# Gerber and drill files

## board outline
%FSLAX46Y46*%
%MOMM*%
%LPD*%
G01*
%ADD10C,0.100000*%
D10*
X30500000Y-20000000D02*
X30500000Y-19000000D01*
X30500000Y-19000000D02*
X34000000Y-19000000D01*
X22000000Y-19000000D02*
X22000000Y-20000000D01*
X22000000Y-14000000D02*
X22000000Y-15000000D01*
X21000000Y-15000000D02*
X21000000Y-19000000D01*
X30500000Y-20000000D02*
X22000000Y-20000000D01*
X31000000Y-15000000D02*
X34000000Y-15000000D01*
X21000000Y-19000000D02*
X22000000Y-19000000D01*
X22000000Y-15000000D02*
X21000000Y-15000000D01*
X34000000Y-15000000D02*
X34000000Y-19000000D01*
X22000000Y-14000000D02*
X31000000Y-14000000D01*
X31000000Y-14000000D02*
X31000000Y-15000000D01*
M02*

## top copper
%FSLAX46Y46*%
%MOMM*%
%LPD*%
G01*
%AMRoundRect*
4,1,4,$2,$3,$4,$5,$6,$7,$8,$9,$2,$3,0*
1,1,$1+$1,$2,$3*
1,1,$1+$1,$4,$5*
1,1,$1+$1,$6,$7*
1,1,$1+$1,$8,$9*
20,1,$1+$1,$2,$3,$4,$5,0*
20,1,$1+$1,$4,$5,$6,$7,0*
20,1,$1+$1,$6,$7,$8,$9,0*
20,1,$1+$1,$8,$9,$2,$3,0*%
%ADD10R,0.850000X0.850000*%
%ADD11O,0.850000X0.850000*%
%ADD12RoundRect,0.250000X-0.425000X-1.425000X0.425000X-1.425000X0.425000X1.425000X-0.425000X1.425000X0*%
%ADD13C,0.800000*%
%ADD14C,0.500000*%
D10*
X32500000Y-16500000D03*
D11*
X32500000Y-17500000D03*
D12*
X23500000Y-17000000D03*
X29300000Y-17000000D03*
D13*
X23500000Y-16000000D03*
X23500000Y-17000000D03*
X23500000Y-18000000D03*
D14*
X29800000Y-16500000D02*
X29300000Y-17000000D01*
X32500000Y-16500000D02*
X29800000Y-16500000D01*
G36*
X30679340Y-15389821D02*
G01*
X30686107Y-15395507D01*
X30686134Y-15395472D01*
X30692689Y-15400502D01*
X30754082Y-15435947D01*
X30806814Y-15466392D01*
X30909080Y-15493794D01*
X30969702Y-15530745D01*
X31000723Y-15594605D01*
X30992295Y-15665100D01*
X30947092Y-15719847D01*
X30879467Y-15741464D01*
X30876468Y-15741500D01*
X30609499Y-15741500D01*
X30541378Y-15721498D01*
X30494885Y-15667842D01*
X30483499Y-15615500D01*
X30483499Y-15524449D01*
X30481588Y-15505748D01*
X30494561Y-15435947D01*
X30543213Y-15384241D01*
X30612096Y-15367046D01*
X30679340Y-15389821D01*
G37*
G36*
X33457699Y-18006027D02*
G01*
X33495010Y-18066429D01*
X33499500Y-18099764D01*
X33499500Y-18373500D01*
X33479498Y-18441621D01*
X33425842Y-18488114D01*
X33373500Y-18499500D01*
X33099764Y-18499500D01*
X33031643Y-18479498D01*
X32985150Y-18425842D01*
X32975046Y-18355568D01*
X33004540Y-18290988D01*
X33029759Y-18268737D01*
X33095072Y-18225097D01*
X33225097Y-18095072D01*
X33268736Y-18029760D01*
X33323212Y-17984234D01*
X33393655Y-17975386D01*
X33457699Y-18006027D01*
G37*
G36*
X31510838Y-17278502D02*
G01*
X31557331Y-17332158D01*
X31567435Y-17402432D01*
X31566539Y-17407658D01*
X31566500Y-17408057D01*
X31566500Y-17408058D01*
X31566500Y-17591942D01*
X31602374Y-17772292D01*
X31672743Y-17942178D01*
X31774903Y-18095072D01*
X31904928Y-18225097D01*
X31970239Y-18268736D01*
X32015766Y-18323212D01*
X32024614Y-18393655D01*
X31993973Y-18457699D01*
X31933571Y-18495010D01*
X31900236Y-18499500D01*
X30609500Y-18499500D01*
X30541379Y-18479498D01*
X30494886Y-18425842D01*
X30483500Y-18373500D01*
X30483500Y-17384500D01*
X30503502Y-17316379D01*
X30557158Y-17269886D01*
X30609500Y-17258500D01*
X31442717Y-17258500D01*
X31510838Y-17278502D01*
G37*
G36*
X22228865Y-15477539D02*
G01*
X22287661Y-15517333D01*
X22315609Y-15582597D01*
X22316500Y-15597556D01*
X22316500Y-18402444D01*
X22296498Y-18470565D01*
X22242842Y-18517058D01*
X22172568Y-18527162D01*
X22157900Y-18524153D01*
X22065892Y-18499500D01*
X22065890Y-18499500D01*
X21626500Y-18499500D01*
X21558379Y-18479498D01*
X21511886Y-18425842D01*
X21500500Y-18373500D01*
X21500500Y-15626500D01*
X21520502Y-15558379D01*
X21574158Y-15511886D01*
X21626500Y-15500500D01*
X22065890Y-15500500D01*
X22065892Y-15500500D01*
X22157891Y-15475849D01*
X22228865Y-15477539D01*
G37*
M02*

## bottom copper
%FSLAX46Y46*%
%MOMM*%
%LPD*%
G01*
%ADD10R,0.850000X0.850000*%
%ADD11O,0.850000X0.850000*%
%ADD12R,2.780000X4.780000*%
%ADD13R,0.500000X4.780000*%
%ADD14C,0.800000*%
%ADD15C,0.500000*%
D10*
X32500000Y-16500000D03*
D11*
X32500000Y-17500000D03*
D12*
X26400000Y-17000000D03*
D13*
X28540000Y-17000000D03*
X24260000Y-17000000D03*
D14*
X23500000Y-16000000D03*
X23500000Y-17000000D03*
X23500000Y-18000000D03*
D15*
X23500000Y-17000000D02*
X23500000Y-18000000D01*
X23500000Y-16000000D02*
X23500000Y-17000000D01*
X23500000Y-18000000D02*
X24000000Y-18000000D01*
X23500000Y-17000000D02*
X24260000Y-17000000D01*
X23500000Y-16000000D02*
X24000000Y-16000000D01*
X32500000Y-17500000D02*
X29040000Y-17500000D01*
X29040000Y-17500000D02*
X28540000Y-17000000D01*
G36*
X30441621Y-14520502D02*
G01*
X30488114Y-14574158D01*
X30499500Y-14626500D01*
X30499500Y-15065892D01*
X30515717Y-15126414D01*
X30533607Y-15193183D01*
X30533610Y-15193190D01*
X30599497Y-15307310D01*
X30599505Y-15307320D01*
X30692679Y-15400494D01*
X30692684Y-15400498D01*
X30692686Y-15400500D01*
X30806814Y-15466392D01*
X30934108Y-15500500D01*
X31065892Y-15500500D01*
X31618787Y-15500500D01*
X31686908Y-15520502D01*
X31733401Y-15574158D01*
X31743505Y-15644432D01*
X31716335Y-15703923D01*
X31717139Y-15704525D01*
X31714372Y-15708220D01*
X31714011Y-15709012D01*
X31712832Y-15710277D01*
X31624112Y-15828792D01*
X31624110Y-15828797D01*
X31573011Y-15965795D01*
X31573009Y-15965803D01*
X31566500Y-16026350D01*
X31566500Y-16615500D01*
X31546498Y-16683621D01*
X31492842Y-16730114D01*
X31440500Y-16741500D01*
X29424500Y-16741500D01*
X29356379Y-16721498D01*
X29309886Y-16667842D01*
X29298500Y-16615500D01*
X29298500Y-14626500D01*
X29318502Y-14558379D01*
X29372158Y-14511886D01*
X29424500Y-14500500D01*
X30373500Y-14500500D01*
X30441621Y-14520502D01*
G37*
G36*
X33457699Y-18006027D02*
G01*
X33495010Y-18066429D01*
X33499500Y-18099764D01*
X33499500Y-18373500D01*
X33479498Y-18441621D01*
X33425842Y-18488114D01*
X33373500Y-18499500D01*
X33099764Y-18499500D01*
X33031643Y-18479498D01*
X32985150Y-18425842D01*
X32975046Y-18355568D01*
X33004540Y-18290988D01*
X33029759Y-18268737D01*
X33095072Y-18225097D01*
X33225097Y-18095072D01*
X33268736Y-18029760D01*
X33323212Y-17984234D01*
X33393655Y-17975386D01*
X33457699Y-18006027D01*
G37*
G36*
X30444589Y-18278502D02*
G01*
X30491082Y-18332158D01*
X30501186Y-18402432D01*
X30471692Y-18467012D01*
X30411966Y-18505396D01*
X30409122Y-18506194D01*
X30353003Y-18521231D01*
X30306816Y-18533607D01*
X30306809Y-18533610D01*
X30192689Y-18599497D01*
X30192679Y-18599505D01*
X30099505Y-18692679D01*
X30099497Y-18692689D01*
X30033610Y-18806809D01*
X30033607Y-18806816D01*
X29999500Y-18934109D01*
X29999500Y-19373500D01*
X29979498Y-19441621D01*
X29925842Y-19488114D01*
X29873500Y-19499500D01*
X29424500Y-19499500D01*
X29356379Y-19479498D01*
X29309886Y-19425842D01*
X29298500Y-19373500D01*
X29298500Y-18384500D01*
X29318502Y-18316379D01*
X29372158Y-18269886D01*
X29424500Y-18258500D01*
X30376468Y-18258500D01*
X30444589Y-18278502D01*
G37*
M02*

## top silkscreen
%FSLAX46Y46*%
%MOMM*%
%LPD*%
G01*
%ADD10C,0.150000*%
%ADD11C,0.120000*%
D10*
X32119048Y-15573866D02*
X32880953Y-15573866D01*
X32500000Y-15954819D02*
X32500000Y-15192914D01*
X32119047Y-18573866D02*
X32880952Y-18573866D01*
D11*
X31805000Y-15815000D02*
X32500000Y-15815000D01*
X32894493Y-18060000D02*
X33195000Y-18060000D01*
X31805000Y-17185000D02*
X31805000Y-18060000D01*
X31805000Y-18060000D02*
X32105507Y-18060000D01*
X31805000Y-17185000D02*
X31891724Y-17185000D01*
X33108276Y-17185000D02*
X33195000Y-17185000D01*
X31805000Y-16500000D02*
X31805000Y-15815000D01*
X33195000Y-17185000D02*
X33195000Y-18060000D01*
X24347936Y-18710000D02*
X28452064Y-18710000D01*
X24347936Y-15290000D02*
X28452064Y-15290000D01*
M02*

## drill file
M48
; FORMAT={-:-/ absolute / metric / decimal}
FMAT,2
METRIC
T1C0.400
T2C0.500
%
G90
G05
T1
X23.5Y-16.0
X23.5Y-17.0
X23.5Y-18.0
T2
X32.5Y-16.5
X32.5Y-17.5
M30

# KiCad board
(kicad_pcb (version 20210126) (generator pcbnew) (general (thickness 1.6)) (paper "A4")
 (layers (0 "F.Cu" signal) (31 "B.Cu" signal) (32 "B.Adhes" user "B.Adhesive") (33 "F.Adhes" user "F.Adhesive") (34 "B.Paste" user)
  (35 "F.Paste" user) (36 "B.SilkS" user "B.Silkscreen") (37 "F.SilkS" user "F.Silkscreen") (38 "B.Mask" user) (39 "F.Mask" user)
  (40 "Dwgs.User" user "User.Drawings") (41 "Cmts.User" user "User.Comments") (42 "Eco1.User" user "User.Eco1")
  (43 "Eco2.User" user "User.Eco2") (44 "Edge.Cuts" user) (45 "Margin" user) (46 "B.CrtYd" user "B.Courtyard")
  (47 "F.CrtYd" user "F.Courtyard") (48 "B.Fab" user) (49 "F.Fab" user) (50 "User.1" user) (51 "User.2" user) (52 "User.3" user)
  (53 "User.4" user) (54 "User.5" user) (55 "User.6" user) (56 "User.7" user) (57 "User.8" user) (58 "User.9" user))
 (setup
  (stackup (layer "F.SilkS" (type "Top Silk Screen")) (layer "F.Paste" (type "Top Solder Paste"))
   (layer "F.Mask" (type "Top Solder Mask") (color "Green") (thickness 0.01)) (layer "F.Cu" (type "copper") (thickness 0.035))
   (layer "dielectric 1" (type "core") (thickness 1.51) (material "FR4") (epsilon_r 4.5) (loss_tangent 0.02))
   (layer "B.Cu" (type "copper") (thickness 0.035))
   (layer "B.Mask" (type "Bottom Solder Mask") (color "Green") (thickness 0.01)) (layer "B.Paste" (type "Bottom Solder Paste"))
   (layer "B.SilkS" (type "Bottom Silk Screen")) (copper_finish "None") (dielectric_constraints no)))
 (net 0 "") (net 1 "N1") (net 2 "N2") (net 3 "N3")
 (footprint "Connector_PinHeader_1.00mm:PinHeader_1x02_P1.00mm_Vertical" (layer "F.Cu") (at 32.5 16.5)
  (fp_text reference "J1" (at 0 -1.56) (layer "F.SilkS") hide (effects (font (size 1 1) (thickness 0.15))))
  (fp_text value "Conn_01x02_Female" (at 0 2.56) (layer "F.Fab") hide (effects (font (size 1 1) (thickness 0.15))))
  (fp_line (start -0.695 -0.685) (end 0 -0.685) (layer "F.SilkS") (width 0.12))
  (fp_line (start 0.394493 1.56) (end 0.695 1.56) (layer "F.SilkS") (width 0.12))
  (fp_line (start -0.695 0.685) (end -0.695 1.56) (layer "F.SilkS") (width 0.12))
  (fp_line (start -0.695 1.56) (end -0.394493 1.56) (layer "F.SilkS") (width 0.12))
  (fp_line (start -0.695 0.685) (end -0.608276 0.685) (layer "F.SilkS") (width 0.12))
  (fp_line (start 0.608276 0.685) (end 0.695 0.685) (layer "F.SilkS") (width 0.12))
  (fp_line (start -0.695 0) (end -0.695 -0.685) (layer "F.SilkS") (width 0.12))
  (fp_line (start 0.695 0.685) (end 0.695 1.56) (layer "F.SilkS") (width 0.12))
  (pad "1" thru_hole rect (at 0 0) (locked) (size 0.85 0.85) (drill 0.5) (layers *.Cu *.Mask) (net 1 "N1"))
  (pad "2" thru_hole oval (at 0 1) (locked) (size 0.85 0.85) (drill 0.5) (layers *.Cu *.Mask) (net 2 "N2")))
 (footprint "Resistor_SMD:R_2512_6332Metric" (layer "F.Cu") (at 26.4 17)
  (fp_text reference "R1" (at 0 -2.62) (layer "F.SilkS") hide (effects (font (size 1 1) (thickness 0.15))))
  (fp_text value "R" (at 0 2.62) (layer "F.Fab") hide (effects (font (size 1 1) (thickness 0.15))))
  (fp_line (start -2.052064 1.71) (end 2.052064 1.71) (layer "F.SilkS") (width 0.12))
  (fp_line (start -2.052064 -1.71) (end 2.052064 -1.71) (layer "F.SilkS") (width 0.12))
  (pad "1" smd roundrect (at -2.9 0) (locked) (size 1.35 3.35) (layers "F.Cu" "F.Paste" "F.Mask") (roundrect_rratio 0.1851851851851852)
   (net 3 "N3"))
  (pad "2" smd roundrect (at 2.9 0) (locked) (size 1.35 3.35) (layers "F.Cu" "F.Paste" "F.Mask") (roundrect_rratio 0.1851851851851852)
   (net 1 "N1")))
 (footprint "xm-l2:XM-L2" (layer "B.Cu") (at 26.4 17 180)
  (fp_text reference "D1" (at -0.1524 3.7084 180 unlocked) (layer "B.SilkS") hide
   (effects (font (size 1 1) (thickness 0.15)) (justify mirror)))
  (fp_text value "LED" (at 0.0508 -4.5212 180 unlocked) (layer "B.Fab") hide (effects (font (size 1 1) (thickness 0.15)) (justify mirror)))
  (pad "" smd rect (at 0 0 180) (locked) (size 2.78 4.78) (layers "B.Cu" "B.Paste" "B.Mask"))
  (pad "1" smd rect (at -2.14 0 180) (locked) (size 0.5 4.78) (layers "B.Cu" "B.Paste" "B.Mask") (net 2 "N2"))
  (pad "2" smd rect (at 2.14 0 180) (locked) (size 0.5 4.78) (layers "B.Cu" "B.Paste" "B.Mask") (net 3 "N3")))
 (gr_line (start 30.5 20) (end 30.5 19) (layer "Edge.Cuts") (width 0.1))
 (gr_line (start 30.5 19) (end 34 19) (layer "Edge.Cuts") (width 0.1))
 (gr_line (start 22 19) (end 22 20) (layer "Edge.Cuts") (width 0.1))
 (gr_line (start 22 14) (end 22 15) (layer "Edge.Cuts") (width 0.1))
 (gr_line (start 21 15) (end 21 19) (layer "Edge.Cuts") (width 0.1))
 (gr_line (start 30.5 20) (end 22 20) (layer "Edge.Cuts") (width 0.1))
 (gr_line (start 31 15) (end 34 15) (layer "Edge.Cuts") (width 0.1))
 (gr_line (start 21 19) (end 22 19) (layer "Edge.Cuts") (width 0.1))
 (gr_line (start 22 15) (end 21 15) (layer "Edge.Cuts") (width 0.1))
 (gr_line (start 34 15) (end 34 19) (layer "Edge.Cuts") (width 0.1))
 (gr_line (start 22 14) (end 31 14) (layer "Edge.Cuts") (width 0.1))
 (gr_line (start 31 14) (end 31 15) (layer "Edge.Cuts") (width 0.1))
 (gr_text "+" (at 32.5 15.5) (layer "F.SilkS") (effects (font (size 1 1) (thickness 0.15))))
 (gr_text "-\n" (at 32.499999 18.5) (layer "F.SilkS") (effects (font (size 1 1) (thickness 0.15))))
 (via (at 23.5 16) (size 0.8) (drill 0.4) (layers "F.Cu" "B.Cu") (free) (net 3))
 (via (at 23.5 17) (size 0.8) (drill 0.4) (layers "F.Cu" "B.Cu") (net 3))
 (via (at 23.5 18) (size 0.8) (drill 0.4) (layers "F.Cu" "B.Cu") (free) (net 3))
 (segment (start 23.5 17) (end 23.5 18) (width 0.5) (layer "B.Cu") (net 3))
 (segment (start 23.5 16) (end 23.5 17) (width 0.5) (layer "B.Cu") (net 3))
 (segment (start 23.5 18) (end 24 18) (width 0.5) (layer "B.Cu") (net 3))
 (segment (start 23.5 17) (end 24.26 17) (width 0.5) (layer "B.Cu") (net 3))
 (segment (start 23.5 16) (end 24 16) (width 0.5) (layer "B.Cu") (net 3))
 (segment (start 32.5 17.5) (end 29.04 17.5) (width 0.5) (layer "B.Cu") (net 2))
 (segment (start 29.04 17.5) (end 28.54 17) (width 0.5) (layer "B.Cu") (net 2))
 (segment (start 29.8 16.5) (end 29.3 17) (width 0.5) (layer "F.Cu") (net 1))
 (segment (start 32.5 16.5) (end 29.8 16.5) (width 0.5) (layer "F.Cu") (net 1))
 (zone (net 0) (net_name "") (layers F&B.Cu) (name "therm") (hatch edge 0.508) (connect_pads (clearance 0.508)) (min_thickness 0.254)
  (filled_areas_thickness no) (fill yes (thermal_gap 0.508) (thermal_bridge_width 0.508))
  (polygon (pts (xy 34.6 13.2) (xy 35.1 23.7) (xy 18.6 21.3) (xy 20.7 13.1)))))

